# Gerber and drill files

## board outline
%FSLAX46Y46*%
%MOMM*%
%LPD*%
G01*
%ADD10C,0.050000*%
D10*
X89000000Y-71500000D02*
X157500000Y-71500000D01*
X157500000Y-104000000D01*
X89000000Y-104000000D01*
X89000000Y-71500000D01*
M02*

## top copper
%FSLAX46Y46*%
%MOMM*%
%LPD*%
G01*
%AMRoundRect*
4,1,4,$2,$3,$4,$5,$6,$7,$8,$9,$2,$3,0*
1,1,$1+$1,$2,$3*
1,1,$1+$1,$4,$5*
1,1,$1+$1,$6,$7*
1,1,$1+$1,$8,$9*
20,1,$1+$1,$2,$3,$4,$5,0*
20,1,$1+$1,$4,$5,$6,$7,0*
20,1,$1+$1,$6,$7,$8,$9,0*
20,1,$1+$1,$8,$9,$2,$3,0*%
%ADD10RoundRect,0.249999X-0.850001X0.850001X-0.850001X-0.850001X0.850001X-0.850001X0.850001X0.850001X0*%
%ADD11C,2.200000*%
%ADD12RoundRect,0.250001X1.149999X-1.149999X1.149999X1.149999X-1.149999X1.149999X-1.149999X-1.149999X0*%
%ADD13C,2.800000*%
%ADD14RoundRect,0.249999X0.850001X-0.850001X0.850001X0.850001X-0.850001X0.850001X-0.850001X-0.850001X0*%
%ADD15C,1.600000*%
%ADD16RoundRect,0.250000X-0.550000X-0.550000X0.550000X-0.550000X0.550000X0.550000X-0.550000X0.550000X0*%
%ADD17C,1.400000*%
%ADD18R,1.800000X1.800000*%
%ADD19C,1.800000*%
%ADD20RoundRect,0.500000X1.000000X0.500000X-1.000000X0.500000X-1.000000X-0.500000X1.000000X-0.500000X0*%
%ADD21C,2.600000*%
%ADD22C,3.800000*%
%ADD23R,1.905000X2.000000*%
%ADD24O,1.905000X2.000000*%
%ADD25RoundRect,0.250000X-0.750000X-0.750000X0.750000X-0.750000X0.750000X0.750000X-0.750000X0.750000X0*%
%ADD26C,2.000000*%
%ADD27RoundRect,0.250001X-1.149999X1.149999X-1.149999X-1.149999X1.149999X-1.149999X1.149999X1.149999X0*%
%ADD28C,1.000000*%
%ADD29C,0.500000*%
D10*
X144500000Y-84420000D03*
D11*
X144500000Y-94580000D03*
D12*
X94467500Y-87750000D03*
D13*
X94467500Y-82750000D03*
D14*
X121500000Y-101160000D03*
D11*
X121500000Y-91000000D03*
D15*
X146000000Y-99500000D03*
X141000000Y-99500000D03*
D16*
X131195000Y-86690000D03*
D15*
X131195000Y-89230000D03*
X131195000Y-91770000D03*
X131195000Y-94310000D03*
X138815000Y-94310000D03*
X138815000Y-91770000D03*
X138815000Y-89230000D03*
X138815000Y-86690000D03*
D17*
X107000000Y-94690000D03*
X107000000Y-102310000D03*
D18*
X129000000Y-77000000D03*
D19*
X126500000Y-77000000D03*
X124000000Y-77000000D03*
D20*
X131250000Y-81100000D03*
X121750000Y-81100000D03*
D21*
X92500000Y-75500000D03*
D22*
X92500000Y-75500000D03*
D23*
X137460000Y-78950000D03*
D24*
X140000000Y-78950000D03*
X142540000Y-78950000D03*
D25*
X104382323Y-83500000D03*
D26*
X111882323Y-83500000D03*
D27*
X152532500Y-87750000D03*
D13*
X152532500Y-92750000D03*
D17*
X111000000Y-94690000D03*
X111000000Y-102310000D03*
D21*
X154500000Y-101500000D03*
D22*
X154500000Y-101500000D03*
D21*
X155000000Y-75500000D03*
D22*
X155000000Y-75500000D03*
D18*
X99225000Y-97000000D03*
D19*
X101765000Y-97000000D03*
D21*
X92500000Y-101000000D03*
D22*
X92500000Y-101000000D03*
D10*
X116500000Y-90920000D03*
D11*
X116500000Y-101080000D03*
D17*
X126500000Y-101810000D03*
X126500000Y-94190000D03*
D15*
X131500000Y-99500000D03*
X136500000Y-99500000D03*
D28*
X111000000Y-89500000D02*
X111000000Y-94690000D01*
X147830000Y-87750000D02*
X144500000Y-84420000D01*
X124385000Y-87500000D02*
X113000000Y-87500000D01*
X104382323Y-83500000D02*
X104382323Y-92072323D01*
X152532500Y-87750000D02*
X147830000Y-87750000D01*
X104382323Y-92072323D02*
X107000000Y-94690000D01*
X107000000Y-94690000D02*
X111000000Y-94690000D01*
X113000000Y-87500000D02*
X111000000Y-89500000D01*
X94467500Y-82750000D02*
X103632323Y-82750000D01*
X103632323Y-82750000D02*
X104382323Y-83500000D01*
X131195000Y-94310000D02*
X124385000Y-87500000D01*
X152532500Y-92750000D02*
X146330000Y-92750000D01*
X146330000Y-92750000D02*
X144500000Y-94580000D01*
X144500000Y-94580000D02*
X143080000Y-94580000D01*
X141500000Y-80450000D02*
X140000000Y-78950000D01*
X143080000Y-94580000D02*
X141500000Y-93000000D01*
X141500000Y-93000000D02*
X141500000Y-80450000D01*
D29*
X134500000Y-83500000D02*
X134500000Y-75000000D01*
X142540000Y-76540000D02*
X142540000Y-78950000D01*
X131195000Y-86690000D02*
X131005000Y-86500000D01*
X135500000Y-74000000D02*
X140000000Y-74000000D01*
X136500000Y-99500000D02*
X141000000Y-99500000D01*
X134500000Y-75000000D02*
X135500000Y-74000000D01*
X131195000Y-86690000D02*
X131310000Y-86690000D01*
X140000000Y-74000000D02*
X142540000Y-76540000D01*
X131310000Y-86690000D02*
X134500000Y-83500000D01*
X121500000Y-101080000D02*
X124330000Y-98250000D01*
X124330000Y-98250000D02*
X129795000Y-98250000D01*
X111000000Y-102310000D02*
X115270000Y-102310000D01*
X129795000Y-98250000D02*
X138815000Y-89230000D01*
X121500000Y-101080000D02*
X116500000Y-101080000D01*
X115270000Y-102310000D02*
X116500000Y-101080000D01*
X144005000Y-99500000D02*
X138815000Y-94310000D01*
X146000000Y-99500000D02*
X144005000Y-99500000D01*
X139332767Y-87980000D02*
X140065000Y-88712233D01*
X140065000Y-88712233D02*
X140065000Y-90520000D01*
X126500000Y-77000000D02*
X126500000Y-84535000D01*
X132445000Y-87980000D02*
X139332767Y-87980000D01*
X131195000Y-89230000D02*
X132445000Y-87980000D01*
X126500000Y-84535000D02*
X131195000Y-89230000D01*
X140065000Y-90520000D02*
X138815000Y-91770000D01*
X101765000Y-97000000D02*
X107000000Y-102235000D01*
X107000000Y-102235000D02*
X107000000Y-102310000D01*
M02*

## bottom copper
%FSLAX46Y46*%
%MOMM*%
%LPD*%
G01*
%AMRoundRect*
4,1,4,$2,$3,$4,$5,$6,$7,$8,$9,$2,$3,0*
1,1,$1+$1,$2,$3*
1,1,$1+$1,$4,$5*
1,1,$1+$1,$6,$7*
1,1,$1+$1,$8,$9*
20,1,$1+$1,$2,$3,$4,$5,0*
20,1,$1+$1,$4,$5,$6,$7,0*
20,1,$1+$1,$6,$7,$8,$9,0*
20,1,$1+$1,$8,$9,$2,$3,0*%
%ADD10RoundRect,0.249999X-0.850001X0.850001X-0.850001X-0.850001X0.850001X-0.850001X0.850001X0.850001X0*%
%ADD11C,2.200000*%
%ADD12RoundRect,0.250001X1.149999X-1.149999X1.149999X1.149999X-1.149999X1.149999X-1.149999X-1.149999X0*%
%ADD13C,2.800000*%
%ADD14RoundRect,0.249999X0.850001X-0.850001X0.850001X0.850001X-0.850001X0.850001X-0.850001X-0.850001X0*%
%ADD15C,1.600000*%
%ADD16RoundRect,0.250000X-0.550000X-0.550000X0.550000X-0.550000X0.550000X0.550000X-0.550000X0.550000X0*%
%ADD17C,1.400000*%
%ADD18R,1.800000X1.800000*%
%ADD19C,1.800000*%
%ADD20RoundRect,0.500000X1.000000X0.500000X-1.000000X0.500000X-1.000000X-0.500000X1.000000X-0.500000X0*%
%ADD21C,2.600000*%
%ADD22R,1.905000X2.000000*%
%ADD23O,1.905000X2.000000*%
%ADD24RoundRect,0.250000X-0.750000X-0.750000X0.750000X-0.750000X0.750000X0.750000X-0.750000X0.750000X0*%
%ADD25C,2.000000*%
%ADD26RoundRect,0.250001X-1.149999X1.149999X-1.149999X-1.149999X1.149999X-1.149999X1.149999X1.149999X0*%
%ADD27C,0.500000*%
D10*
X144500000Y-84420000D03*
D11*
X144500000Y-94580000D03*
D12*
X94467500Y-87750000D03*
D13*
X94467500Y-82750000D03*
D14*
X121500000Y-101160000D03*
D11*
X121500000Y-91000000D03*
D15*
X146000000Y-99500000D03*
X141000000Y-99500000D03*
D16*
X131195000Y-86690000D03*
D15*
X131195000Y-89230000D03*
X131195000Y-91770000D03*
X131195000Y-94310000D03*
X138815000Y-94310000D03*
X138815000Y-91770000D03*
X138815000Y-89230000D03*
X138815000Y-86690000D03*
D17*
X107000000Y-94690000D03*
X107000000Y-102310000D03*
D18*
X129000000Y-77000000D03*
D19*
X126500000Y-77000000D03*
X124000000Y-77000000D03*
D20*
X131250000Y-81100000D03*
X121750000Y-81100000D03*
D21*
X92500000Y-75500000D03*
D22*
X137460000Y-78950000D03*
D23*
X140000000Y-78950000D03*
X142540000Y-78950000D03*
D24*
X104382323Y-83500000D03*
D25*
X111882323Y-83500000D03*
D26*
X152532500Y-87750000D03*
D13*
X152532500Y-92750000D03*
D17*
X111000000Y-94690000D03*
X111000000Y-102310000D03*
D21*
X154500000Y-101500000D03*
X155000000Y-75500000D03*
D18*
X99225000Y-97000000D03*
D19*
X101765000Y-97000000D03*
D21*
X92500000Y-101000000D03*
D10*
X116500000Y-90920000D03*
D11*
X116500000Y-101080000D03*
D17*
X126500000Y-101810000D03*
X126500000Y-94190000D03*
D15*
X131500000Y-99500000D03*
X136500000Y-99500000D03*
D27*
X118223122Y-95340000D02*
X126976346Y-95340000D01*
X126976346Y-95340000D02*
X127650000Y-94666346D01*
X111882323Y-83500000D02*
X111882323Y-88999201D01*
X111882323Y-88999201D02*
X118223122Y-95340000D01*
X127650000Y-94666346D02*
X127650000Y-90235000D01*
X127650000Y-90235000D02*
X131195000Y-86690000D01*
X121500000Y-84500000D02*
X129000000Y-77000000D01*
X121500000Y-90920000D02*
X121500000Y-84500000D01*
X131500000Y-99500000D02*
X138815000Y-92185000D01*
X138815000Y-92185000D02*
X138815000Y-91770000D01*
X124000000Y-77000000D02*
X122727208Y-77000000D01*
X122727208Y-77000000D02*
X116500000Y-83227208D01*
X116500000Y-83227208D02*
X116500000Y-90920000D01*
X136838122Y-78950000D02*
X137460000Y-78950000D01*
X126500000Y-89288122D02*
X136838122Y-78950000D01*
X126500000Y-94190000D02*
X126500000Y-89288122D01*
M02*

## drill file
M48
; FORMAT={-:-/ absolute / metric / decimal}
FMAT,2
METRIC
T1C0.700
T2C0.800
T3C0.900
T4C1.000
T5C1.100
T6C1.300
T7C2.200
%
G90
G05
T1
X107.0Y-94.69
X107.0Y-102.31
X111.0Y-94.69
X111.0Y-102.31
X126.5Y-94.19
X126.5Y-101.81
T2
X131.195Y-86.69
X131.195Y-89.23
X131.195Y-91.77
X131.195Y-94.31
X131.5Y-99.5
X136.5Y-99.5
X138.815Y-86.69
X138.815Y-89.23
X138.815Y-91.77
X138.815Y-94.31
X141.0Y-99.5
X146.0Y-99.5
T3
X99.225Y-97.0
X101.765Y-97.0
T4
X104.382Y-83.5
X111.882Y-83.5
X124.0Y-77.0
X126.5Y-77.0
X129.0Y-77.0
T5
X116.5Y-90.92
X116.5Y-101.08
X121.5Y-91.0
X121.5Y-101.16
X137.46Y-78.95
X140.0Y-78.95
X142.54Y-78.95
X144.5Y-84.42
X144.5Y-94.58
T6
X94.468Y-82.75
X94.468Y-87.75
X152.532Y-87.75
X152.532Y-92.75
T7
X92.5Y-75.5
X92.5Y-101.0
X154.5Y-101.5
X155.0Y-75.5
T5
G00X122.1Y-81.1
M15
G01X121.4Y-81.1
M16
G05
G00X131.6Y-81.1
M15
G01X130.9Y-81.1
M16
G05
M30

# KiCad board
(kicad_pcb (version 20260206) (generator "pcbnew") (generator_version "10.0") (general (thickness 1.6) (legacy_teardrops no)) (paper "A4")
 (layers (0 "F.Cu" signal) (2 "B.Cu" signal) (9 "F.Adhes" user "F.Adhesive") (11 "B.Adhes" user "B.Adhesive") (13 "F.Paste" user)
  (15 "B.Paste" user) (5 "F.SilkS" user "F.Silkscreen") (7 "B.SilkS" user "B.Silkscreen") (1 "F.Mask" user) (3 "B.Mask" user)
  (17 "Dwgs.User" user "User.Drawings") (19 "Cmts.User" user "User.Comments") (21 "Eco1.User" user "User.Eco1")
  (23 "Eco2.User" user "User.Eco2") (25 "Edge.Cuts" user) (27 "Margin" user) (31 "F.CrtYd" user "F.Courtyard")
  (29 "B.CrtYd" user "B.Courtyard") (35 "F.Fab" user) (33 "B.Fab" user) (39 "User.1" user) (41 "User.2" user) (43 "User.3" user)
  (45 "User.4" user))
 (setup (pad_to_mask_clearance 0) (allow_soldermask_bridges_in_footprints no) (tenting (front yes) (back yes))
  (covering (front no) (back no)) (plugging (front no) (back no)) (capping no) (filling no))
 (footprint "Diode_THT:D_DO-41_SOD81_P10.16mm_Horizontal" (layer "F.Cu") (at 144.5 84.42 -90)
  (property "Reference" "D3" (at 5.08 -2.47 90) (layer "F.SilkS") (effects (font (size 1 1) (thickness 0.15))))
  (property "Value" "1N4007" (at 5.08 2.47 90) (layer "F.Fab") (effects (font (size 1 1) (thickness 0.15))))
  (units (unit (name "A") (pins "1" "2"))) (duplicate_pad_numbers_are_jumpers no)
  (pad "1" thru_hole roundrect (at 0 0 270) (size 2.2 2.2) (drill 1.1) (layers "*.Cu" "*.Mask") (remove_unused_layers no)
   (roundrect_rratio 0.113636) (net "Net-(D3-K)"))
  (pad "2" thru_hole circle (at 10.16 0 270) (size 2.2 2.2) (drill 1.1) (layers "*.Cu" "*.Mask") (remove_unused_layers no)
   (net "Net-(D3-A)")))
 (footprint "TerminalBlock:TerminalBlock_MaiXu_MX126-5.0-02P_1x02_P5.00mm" (layer "F.Cu") (at 94.4675 87.75 90)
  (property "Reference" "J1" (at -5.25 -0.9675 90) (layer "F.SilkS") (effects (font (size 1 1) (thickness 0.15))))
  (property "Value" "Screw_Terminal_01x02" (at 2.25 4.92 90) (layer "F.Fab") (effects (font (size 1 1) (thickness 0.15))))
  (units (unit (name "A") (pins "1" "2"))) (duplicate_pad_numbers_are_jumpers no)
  (pad "1" thru_hole roundrect (at 0 0 90) (size 2.8 2.8) (drill 1.3) (layers "*.Cu" "*.Mask") (remove_unused_layers no)
   (roundrect_rratio 0.089286) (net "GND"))
  (pad "2" thru_hole circle (at 5 0 90) (size 2.8 2.8) (drill 1.3) (layers "*.Cu" "*.Mask") (remove_unused_layers no) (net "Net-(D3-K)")))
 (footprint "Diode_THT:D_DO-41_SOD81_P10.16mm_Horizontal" (layer "F.Cu") (at 121.5 101.16 90)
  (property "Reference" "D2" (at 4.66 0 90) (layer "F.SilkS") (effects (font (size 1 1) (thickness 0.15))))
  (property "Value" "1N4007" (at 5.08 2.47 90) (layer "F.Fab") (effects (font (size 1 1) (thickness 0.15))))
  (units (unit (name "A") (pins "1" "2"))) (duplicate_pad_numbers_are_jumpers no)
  (pad "1" thru_hole roundrect (at 0 0 90) (size 2.2 2.2) (drill 1.1) (layers "*.Cu" "*.Mask") (remove_unused_layers no)
   (roundrect_rratio 0.113636) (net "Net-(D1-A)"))
  (pad "2" thru_hole circle (at 10.16 0 90) (size 2.2 2.2) (drill 1.1) (layers "*.Cu" "*.Mask") (remove_unused_layers no) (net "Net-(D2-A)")))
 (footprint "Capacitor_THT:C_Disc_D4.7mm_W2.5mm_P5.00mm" (layer "F.Cu") (at 146 99.5 180)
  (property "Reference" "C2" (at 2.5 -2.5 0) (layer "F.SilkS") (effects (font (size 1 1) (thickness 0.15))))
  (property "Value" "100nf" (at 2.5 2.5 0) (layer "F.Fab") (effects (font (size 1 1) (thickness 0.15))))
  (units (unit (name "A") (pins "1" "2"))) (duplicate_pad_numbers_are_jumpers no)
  (pad "1" thru_hole circle (at 0 0 180) (size 1.6 1.6) (drill 0.8) (layers "*.Cu" "*.Mask") (remove_unused_layers no) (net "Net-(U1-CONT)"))
  (pad "2" thru_hole circle (at 5 0 180) (size 1.6 1.6) (drill 0.8) (layers "*.Cu" "*.Mask") (remove_unused_layers no) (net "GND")))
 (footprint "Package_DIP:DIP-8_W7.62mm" (layer "F.Cu") (at 131.195 86.69)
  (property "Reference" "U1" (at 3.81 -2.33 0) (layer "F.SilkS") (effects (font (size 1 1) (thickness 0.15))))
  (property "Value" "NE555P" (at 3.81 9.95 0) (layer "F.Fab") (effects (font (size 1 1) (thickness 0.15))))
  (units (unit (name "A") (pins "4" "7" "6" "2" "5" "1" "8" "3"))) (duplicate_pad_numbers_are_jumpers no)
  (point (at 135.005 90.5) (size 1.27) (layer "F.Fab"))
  (pad "1" thru_hole roundrect (at 0 0) (size 1.6 1.6) (drill 0.8) (layers "*.Cu" "*.Mask") (remove_unused_layers no)
   (roundrect_rratio 0.15625) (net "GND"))
  (pad "2" thru_hole circle (at 0 2.54) (size 1.6 1.6) (drill 0.8) (layers "*.Cu" "*.Mask") (remove_unused_layers no) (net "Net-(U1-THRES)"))
  (pad "3" thru_hole circle (at 0 5.08) (size 1.6 1.6) (drill 0.8) (layers "*.Cu" "*.Mask") (remove_unused_layers no) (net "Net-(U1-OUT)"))
  (pad "4" thru_hole circle (at 0 7.62) (size 1.6 1.6) (drill 0.8) (layers "*.Cu" "*.Mask") (remove_unused_layers no) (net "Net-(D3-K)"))
  (pad "5" thru_hole circle (at 7.62 7.62) (size 1.6 1.6) (drill 0.8) (layers "*.Cu" "*.Mask") (remove_unused_layers no)
   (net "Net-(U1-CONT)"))
  (pad "6" thru_hole circle (at 7.62 5.08) (size 1.6 1.6) (drill 0.8) (layers "*.Cu" "*.Mask") (remove_unused_layers no)
   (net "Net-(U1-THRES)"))
  (pad "7" thru_hole circle (at 7.62 2.54) (size 1.6 1.6) (drill 0.8) (layers "*.Cu" "*.Mask") (remove_unused_layers no) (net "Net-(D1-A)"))
  (pad "8" thru_hole circle (at 7.62 0) (size 1.6 1.6) (drill 0.8) (layers "*.Cu" "*.Mask") (remove_unused_layers no) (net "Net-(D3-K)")))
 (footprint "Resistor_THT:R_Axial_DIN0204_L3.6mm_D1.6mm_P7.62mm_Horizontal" (layer "F.Cu") (at 107 94.69 -90)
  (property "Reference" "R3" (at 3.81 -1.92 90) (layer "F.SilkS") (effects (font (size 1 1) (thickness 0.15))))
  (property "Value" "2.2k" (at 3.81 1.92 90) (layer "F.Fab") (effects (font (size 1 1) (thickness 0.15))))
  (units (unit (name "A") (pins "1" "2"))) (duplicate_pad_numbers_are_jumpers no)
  (pad "1" thru_hole circle (at 0 0 270) (size 1.4 1.4) (drill 0.7) (layers "*.Cu" "*.Mask") (remove_unused_layers no) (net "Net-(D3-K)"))
  (pad "2" thru_hole circle (at 7.62 0 270) (size 1.4 1.4) (drill 0.7) (layers "*.Cu" "*.Mask") (remove_unused_layers no) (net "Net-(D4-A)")))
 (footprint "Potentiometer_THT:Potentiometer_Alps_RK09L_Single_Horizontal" (layer "F.Cu") (at 129 77 -90)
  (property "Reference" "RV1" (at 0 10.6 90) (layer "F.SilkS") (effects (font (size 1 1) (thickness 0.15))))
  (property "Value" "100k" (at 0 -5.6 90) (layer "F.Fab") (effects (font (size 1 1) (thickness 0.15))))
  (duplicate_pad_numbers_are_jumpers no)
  (pad "1" thru_hole rect (at 0 0 90) (size 1.8 1.8) (drill 1) (layers "*.Cu" "*.Mask") (remove_unused_layers no) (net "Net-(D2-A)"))
  (pad "2" thru_hole circle (at 0 2.5 90) (size 1.8 1.8) (drill 1) (layers "*.Cu" "*.Mask") (remove_unused_layers no) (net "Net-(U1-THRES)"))
  (pad "3" thru_hole circle (at 0 5 90) (size 1.8 1.8) (drill 1) (layers "*.Cu" "*.Mask") (remove_unused_layers no) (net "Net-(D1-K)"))
  (pad "MP" thru_hole roundrect (at 4.1 -2.25 180) (size 3 2) (drill oval 1.8 1.1) (layers "*.Cu" "*.Mask") (remove_unused_layers no)
   (roundrect_rratio 0.25))
  (pad "MP" thru_hole roundrect (at 4.1 7.25 180) (size 3 2) (drill oval 1.8 1.1) (layers "*.Cu" "*.Mask") (remove_unused_layers no)
   (roundrect_rratio 0.25)))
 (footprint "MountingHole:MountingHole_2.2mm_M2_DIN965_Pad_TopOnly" (layer "F.Cu") (at 92.5 75.5)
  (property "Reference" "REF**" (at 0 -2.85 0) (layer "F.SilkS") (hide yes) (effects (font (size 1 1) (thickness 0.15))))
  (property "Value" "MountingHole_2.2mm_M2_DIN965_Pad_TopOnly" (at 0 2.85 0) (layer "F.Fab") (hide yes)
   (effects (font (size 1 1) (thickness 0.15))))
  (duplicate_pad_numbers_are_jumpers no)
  (pad "1" thru_hole circle (at 0 0) (size 2.6 2.6) (drill 2.2) (layers "*.Cu" "*.Mask") (remove_unused_layers no) (zone_connect 2))
  (pad "1" connect circle (at 0 0) (size 3.8 3.8) (layers "F.Cu" "F.Mask") (zone_connect 2)))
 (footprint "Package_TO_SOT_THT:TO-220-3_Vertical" (layer "F.Cu") (at 137.46 78.95)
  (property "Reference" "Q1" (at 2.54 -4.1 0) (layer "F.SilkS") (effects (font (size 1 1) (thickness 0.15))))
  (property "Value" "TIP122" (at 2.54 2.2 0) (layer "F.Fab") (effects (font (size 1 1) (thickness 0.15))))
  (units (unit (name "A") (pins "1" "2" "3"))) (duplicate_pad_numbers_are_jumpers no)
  (pad "1" thru_hole rect (at 0 0) (size 1.905 2) (drill 1.1) (layers "*.Cu" "*.Mask") (remove_unused_layers no) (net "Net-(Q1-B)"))
  (pad "2" thru_hole oval (at 2.54 0) (size 1.905 2) (drill 1.1) (layers "*.Cu" "*.Mask") (remove_unused_layers no) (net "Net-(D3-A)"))
  (pad "3" thru_hole oval (at 5.08 0) (size 1.905 2) (drill 1.1) (layers "*.Cu" "*.Mask") (remove_unused_layers no) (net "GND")))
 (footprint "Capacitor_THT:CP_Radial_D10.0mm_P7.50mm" (layer "F.Cu") (at 104.382323 83.5)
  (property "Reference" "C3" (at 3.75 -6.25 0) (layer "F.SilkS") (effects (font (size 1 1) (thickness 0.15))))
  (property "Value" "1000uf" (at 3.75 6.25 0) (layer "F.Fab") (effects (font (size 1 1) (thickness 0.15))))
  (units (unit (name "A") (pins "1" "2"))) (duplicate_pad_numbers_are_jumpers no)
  (pad "1" thru_hole roundrect (at 0 0) (size 2 2) (drill 1) (layers "*.Cu" "*.Mask") (remove_unused_layers no) (roundrect_rratio 0.125)
   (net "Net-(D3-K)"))
  (pad "2" thru_hole circle (at 7.5 0) (size 2 2) (drill 1) (layers "*.Cu" "*.Mask") (remove_unused_layers no) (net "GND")))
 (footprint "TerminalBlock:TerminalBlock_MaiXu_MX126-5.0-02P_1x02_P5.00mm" (layer "F.Cu") (at 152.5325 87.75 -90)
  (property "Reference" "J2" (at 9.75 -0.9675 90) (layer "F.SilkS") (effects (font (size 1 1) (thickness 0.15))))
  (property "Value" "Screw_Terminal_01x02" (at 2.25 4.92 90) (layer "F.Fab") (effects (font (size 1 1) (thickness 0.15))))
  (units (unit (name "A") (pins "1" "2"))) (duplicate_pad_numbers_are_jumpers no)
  (pad "1" thru_hole roundrect (at 0 0 270) (size 2.8 2.8) (drill 1.3) (layers "*.Cu" "*.Mask") (remove_unused_layers no)
   (roundrect_rratio 0.089286) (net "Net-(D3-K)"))
  (pad "2" thru_hole circle (at 5 0 270) (size 2.8 2.8) (drill 1.3) (layers "*.Cu" "*.Mask") (remove_unused_layers no) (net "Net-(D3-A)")))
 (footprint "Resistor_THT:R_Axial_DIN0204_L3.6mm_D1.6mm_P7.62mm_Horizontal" (layer "F.Cu") (at 111 94.69 -90)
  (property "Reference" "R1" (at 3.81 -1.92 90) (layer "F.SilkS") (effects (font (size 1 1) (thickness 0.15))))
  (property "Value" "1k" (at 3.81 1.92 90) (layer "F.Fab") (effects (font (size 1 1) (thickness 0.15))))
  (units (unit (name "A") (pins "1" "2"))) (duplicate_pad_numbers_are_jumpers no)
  (pad "1" thru_hole circle (at 0 0 270) (size 1.4 1.4) (drill 0.7) (layers "*.Cu" "*.Mask") (remove_unused_layers no) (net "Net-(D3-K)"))
  (pad "2" thru_hole circle (at 7.62 0 270) (size 1.4 1.4) (drill 0.7) (layers "*.Cu" "*.Mask") (remove_unused_layers no) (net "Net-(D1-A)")))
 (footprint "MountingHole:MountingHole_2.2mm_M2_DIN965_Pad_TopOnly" (layer "F.Cu") (at 154.5 101.5)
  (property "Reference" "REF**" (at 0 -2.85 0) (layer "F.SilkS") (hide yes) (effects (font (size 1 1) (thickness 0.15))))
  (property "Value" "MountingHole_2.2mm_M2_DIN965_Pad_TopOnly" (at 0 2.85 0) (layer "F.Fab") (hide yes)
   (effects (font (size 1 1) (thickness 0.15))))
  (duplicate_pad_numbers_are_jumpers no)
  (pad "1" thru_hole circle (at 0 0) (size 2.6 2.6) (drill 2.2) (layers "*.Cu" "*.Mask") (remove_unused_layers no) (zone_connect 2))
  (pad "1" connect circle (at 0 0) (size 3.8 3.8) (layers "F.Cu" "F.Mask") (zone_connect 2)))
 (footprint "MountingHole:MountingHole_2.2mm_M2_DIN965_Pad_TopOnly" (layer "F.Cu") (at 155 75.5)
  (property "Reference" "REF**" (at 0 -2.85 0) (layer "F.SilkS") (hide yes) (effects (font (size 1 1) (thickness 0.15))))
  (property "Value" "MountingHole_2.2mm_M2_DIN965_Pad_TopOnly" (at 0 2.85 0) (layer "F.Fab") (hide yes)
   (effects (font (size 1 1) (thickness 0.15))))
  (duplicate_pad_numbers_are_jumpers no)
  (pad "1" thru_hole circle (at 0 0) (size 2.6 2.6) (drill 2.2) (layers "*.Cu" "*.Mask") (remove_unused_layers no) (zone_connect 2))
  (pad "1" connect circle (at 0 0) (size 3.8 3.8) (layers "F.Cu" "F.Mask") (zone_connect 2)))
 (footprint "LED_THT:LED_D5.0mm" (layer "F.Cu") (at 99.225 97)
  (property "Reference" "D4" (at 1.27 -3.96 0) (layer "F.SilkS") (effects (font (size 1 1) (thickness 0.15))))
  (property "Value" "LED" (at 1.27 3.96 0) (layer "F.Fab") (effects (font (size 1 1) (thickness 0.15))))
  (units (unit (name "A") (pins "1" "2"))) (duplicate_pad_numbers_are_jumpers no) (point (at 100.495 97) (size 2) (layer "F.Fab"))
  (pad "1" thru_hole rect (at 0 0) (size 1.8 1.8) (drill 0.9) (layers "*.Cu" "*.Mask") (remove_unused_layers no) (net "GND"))
  (pad "2" thru_hole circle (at 2.54 0) (size 1.8 1.8) (drill 0.9) (layers "*.Cu" "*.Mask") (remove_unused_layers no) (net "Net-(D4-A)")))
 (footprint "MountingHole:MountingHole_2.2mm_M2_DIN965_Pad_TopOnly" (layer "F.Cu") (at 92.5 101)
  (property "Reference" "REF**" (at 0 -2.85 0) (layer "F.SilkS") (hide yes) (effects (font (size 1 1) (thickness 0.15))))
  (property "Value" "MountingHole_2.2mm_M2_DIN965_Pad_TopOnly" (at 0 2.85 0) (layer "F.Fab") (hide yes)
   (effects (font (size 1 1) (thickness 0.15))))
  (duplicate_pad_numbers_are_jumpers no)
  (pad "1" thru_hole circle (at 0 0) (size 2.6 2.6) (drill 2.2) (layers "*.Cu" "*.Mask") (remove_unused_layers no) (zone_connect 2))
  (pad "1" connect circle (at 0 0) (size 3.8 3.8) (layers "F.Cu" "F.Mask") (zone_connect 2)))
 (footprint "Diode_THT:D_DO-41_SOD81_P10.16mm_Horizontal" (layer "F.Cu") (at 116.5 90.92 -90)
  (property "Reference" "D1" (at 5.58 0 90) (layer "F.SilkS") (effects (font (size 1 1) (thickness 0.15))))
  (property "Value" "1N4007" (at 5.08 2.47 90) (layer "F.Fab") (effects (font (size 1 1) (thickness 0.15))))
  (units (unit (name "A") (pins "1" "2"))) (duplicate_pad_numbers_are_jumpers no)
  (pad "1" thru_hole roundrect (at 0 0 270) (size 2.2 2.2) (drill 1.1) (layers "*.Cu" "*.Mask") (remove_unused_layers no)
   (roundrect_rratio 0.113636) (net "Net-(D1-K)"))
  (pad "2" thru_hole circle (at 10.16 0 270) (size 2.2 2.2) (drill 1.1) (layers "*.Cu" "*.Mask") (remove_unused_layers no)
   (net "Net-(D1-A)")))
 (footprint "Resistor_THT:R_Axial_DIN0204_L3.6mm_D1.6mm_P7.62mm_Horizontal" (layer "F.Cu") (at 126.5 101.81 90)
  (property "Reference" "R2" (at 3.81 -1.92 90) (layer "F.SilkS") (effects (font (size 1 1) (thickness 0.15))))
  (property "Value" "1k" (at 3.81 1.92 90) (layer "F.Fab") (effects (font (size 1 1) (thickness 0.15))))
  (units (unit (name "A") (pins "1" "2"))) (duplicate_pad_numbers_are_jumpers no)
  (pad "1" thru_hole circle (at 0 0 90) (size 1.4 1.4) (drill 0.7) (layers "*.Cu" "*.Mask") (remove_unused_layers no) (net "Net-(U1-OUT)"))
  (pad "2" thru_hole circle (at 7.62 0 90) (size 1.4 1.4) (drill 0.7) (layers "*.Cu" "*.Mask") (remove_unused_layers no) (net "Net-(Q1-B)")))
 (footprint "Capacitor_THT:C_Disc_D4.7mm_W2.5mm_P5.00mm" (layer "F.Cu") (at 131.5 99.5)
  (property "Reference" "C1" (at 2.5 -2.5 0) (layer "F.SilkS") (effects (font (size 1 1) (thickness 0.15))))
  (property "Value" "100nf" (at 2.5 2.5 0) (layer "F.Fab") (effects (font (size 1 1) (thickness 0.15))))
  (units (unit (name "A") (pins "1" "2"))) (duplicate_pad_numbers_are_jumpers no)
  (pad "1" thru_hole circle (at 0 0) (size 1.6 1.6) (drill 0.8) (layers "*.Cu" "*.Mask") (remove_unused_layers no) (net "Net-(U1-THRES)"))
  (pad "2" thru_hole circle (at 5 0) (size 1.6 1.6) (drill 0.8) (layers "*.Cu" "*.Mask") (remove_unused_layers no) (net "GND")))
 (gr_rect (start 89 71.5) (end 157.5 104) (stroke (width 0.05) (type default)) (fill no) (layer "Edge.Cuts"))
 (segment (start 111 89.5) (end 111 94.69) (width 1) (layer "F.Cu") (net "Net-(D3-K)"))
 (segment (start 147.83 87.75) (end 144.5 84.42) (width 1) (layer "F.Cu") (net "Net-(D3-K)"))
 (segment (start 124.385 87.5) (end 113 87.5) (width 1) (layer "F.Cu") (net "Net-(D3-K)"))
 (segment (start 104.382323 83.5) (end 104.382323 92.072323) (width 1) (layer "F.Cu") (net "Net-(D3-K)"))
 (segment (start 152.5325 87.75) (end 147.83 87.75) (width 1) (layer "F.Cu") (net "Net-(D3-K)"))
 (segment (start 104.382323 92.072323) (end 107 94.69) (width 1) (layer "F.Cu") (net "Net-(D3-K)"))
 (segment (start 107 94.69) (end 111 94.69) (width 1) (layer "F.Cu") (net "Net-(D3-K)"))
 (segment (start 113 87.5) (end 111 89.5) (width 1) (layer "F.Cu") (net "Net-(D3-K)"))
 (segment (start 94.4675 82.75) (end 103.632323 82.75) (width 1) (layer "F.Cu") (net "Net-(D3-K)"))
 (segment (start 103.632323 82.75) (end 104.382323 83.5) (width 1) (layer "F.Cu") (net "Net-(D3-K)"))
 (segment (start 131.195 94.31) (end 124.385 87.5) (width 1) (layer "F.Cu") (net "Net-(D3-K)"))
 (segment (start 152.5325 92.75) (end 146.33 92.75) (width 1) (layer "F.Cu") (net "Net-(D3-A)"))
 (segment (start 146.33 92.75) (end 144.5 94.58) (width 1) (layer "F.Cu") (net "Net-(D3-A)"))
 (segment (start 144.5 94.58) (end 143.08 94.58) (width 1) (layer "F.Cu") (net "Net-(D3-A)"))
 (segment (start 141.5 80.45) (end 140 78.95) (width 1) (layer "F.Cu") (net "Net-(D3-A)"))
 (segment (start 143.08 94.58) (end 141.5 93) (width 1) (layer "F.Cu") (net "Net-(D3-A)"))
 (segment (start 141.5 93) (end 141.5 80.45) (width 1) (layer "F.Cu") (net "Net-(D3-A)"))
 (segment (start 134.5 83.5) (end 134.5 75) (width 0.5) (layer "F.Cu") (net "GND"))
 (segment (start 142.54 76.54) (end 142.54 78.95) (width 0.5) (layer "F.Cu") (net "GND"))
 (segment (start 131.195 86.69) (end 131.005 86.5) (width 0.5) (layer "F.Cu") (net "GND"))
 (segment (start 135.5 74) (end 140 74) (width 0.5) (layer "F.Cu") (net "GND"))
 (segment (start 136.5 99.5) (end 141 99.5) (width 0.5) (layer "F.Cu") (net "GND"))
 (segment (start 134.5 75) (end 135.5 74) (width 0.5) (layer "F.Cu") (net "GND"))
 (segment (start 131.195 86.69) (end 131.31 86.69) (width 0.5) (layer "F.Cu") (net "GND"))
 (segment (start 140 74) (end 142.54 76.54) (width 0.5) (layer "F.Cu") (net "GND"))
 (segment (start 131.31 86.69) (end 134.5 83.5) (width 0.5) (layer "F.Cu") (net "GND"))
 (segment (start 118.223122 95.34) (end 126.976346 95.34) (width 0.5) (layer "B.Cu") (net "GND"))
 (segment (start 126.976346 95.34) (end 127.65 94.666346) (width 0.5) (layer "B.Cu") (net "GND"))
 (segment (start 111.882323 83.5) (end 111.882323 88.999201) (width 0.5) (layer "B.Cu") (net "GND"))
 (segment (start 111.882323 88.999201) (end 118.223122 95.34) (width 0.5) (layer "B.Cu") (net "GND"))
 (segment (start 127.65 94.666346) (end 127.65 90.235) (width 0.5) (layer "B.Cu") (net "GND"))
 (segment (start 127.65 90.235) (end 131.195 86.69) (width 0.5) (layer "B.Cu") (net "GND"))
 (segment (start 121.5 101.08) (end 124.33 98.25) (width 0.5) (layer "F.Cu") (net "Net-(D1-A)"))
 (segment (start 124.33 98.25) (end 129.795 98.25) (width 0.5) (layer "F.Cu") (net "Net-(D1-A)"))
 (segment (start 111 102.31) (end 115.27 102.31) (width 0.5) (layer "F.Cu") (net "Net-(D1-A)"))
 (segment (start 129.795 98.25) (end 138.815 89.23) (width 0.5) (layer "F.Cu") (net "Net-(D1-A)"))
 (segment (start 121.5 101.08) (end 116.5 101.08) (width 0.5) (layer "F.Cu") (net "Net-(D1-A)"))
 (segment (start 115.27 102.31) (end 116.5 101.08) (width 0.5) (layer "F.Cu") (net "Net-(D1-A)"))
 (segment (start 121.5 84.5) (end 129 77) (width 0.5) (layer "B.Cu") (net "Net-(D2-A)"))
 (segment (start 121.5 90.92) (end 121.5 84.5) (width 0.5) (layer "B.Cu") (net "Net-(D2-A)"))
 (segment (start 144.005 99.5) (end 138.815 94.31) (width 0.5) (layer "F.Cu") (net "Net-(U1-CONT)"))
 (segment (start 146 99.5) (end 144.005 99.5) (width 0.5) (layer "F.Cu") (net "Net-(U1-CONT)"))
 (segment (start 139.332767 87.98) (end 140.065 88.712233) (width 0.5) (layer "F.Cu") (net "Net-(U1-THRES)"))
 (segment (start 140.065 88.712233) (end 140.065 90.52) (width 0.5) (layer "F.Cu") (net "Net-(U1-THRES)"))
 (segment (start 126.5 77) (end 126.5 84.535) (width 0.5) (layer "F.Cu") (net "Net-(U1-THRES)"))
 (segment (start 132.445 87.98) (end 139.332767 87.98) (width 0.5) (layer "F.Cu") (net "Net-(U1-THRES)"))
 (segment (start 131.195 89.23) (end 132.445 87.98) (width 0.5) (layer "F.Cu") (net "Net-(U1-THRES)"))
 (segment (start 126.5 84.535) (end 131.195 89.23) (width 0.5) (layer "F.Cu") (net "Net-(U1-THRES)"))
 (segment (start 140.065 90.52) (end 138.815 91.77) (width 0.5) (layer "F.Cu") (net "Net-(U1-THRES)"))
 (segment (start 131.5 99.5) (end 138.815 92.185) (width 0.5) (layer "B.Cu") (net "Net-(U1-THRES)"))
 (segment (start 138.815 92.185) (end 138.815 91.77) (width 0.5) (layer "B.Cu") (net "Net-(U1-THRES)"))
 (segment (start 101.765 97) (end 107 102.235) (width 0.5) (layer "F.Cu") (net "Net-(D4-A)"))
 (segment (start 107 102.235) (end 107 102.31) (width 0.5) (layer "F.Cu") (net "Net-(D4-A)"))
 (segment (start 124 77) (end 122.727208 77) (width 0.5) (layer "B.Cu") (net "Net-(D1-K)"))
 (segment (start 122.727208 77) (end 116.5 83.227208) (width 0.5) (layer "B.Cu") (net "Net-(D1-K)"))
 (segment (start 116.5 83.227208) (end 116.5 90.92) (width 0.5) (layer "B.Cu") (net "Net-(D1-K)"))
 (segment (start 136.838122 78.95) (end 137.46 78.95) (width 0.5) (layer "B.Cu") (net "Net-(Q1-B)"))
 (segment (start 126.5 89.288122) (end 136.838122 78.95) (width 0.5) (layer "B.Cu") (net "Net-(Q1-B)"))
 (segment (start 126.5 94.19) (end 126.5 89.288122) (width 0.5) (layer "B.Cu") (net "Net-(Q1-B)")))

